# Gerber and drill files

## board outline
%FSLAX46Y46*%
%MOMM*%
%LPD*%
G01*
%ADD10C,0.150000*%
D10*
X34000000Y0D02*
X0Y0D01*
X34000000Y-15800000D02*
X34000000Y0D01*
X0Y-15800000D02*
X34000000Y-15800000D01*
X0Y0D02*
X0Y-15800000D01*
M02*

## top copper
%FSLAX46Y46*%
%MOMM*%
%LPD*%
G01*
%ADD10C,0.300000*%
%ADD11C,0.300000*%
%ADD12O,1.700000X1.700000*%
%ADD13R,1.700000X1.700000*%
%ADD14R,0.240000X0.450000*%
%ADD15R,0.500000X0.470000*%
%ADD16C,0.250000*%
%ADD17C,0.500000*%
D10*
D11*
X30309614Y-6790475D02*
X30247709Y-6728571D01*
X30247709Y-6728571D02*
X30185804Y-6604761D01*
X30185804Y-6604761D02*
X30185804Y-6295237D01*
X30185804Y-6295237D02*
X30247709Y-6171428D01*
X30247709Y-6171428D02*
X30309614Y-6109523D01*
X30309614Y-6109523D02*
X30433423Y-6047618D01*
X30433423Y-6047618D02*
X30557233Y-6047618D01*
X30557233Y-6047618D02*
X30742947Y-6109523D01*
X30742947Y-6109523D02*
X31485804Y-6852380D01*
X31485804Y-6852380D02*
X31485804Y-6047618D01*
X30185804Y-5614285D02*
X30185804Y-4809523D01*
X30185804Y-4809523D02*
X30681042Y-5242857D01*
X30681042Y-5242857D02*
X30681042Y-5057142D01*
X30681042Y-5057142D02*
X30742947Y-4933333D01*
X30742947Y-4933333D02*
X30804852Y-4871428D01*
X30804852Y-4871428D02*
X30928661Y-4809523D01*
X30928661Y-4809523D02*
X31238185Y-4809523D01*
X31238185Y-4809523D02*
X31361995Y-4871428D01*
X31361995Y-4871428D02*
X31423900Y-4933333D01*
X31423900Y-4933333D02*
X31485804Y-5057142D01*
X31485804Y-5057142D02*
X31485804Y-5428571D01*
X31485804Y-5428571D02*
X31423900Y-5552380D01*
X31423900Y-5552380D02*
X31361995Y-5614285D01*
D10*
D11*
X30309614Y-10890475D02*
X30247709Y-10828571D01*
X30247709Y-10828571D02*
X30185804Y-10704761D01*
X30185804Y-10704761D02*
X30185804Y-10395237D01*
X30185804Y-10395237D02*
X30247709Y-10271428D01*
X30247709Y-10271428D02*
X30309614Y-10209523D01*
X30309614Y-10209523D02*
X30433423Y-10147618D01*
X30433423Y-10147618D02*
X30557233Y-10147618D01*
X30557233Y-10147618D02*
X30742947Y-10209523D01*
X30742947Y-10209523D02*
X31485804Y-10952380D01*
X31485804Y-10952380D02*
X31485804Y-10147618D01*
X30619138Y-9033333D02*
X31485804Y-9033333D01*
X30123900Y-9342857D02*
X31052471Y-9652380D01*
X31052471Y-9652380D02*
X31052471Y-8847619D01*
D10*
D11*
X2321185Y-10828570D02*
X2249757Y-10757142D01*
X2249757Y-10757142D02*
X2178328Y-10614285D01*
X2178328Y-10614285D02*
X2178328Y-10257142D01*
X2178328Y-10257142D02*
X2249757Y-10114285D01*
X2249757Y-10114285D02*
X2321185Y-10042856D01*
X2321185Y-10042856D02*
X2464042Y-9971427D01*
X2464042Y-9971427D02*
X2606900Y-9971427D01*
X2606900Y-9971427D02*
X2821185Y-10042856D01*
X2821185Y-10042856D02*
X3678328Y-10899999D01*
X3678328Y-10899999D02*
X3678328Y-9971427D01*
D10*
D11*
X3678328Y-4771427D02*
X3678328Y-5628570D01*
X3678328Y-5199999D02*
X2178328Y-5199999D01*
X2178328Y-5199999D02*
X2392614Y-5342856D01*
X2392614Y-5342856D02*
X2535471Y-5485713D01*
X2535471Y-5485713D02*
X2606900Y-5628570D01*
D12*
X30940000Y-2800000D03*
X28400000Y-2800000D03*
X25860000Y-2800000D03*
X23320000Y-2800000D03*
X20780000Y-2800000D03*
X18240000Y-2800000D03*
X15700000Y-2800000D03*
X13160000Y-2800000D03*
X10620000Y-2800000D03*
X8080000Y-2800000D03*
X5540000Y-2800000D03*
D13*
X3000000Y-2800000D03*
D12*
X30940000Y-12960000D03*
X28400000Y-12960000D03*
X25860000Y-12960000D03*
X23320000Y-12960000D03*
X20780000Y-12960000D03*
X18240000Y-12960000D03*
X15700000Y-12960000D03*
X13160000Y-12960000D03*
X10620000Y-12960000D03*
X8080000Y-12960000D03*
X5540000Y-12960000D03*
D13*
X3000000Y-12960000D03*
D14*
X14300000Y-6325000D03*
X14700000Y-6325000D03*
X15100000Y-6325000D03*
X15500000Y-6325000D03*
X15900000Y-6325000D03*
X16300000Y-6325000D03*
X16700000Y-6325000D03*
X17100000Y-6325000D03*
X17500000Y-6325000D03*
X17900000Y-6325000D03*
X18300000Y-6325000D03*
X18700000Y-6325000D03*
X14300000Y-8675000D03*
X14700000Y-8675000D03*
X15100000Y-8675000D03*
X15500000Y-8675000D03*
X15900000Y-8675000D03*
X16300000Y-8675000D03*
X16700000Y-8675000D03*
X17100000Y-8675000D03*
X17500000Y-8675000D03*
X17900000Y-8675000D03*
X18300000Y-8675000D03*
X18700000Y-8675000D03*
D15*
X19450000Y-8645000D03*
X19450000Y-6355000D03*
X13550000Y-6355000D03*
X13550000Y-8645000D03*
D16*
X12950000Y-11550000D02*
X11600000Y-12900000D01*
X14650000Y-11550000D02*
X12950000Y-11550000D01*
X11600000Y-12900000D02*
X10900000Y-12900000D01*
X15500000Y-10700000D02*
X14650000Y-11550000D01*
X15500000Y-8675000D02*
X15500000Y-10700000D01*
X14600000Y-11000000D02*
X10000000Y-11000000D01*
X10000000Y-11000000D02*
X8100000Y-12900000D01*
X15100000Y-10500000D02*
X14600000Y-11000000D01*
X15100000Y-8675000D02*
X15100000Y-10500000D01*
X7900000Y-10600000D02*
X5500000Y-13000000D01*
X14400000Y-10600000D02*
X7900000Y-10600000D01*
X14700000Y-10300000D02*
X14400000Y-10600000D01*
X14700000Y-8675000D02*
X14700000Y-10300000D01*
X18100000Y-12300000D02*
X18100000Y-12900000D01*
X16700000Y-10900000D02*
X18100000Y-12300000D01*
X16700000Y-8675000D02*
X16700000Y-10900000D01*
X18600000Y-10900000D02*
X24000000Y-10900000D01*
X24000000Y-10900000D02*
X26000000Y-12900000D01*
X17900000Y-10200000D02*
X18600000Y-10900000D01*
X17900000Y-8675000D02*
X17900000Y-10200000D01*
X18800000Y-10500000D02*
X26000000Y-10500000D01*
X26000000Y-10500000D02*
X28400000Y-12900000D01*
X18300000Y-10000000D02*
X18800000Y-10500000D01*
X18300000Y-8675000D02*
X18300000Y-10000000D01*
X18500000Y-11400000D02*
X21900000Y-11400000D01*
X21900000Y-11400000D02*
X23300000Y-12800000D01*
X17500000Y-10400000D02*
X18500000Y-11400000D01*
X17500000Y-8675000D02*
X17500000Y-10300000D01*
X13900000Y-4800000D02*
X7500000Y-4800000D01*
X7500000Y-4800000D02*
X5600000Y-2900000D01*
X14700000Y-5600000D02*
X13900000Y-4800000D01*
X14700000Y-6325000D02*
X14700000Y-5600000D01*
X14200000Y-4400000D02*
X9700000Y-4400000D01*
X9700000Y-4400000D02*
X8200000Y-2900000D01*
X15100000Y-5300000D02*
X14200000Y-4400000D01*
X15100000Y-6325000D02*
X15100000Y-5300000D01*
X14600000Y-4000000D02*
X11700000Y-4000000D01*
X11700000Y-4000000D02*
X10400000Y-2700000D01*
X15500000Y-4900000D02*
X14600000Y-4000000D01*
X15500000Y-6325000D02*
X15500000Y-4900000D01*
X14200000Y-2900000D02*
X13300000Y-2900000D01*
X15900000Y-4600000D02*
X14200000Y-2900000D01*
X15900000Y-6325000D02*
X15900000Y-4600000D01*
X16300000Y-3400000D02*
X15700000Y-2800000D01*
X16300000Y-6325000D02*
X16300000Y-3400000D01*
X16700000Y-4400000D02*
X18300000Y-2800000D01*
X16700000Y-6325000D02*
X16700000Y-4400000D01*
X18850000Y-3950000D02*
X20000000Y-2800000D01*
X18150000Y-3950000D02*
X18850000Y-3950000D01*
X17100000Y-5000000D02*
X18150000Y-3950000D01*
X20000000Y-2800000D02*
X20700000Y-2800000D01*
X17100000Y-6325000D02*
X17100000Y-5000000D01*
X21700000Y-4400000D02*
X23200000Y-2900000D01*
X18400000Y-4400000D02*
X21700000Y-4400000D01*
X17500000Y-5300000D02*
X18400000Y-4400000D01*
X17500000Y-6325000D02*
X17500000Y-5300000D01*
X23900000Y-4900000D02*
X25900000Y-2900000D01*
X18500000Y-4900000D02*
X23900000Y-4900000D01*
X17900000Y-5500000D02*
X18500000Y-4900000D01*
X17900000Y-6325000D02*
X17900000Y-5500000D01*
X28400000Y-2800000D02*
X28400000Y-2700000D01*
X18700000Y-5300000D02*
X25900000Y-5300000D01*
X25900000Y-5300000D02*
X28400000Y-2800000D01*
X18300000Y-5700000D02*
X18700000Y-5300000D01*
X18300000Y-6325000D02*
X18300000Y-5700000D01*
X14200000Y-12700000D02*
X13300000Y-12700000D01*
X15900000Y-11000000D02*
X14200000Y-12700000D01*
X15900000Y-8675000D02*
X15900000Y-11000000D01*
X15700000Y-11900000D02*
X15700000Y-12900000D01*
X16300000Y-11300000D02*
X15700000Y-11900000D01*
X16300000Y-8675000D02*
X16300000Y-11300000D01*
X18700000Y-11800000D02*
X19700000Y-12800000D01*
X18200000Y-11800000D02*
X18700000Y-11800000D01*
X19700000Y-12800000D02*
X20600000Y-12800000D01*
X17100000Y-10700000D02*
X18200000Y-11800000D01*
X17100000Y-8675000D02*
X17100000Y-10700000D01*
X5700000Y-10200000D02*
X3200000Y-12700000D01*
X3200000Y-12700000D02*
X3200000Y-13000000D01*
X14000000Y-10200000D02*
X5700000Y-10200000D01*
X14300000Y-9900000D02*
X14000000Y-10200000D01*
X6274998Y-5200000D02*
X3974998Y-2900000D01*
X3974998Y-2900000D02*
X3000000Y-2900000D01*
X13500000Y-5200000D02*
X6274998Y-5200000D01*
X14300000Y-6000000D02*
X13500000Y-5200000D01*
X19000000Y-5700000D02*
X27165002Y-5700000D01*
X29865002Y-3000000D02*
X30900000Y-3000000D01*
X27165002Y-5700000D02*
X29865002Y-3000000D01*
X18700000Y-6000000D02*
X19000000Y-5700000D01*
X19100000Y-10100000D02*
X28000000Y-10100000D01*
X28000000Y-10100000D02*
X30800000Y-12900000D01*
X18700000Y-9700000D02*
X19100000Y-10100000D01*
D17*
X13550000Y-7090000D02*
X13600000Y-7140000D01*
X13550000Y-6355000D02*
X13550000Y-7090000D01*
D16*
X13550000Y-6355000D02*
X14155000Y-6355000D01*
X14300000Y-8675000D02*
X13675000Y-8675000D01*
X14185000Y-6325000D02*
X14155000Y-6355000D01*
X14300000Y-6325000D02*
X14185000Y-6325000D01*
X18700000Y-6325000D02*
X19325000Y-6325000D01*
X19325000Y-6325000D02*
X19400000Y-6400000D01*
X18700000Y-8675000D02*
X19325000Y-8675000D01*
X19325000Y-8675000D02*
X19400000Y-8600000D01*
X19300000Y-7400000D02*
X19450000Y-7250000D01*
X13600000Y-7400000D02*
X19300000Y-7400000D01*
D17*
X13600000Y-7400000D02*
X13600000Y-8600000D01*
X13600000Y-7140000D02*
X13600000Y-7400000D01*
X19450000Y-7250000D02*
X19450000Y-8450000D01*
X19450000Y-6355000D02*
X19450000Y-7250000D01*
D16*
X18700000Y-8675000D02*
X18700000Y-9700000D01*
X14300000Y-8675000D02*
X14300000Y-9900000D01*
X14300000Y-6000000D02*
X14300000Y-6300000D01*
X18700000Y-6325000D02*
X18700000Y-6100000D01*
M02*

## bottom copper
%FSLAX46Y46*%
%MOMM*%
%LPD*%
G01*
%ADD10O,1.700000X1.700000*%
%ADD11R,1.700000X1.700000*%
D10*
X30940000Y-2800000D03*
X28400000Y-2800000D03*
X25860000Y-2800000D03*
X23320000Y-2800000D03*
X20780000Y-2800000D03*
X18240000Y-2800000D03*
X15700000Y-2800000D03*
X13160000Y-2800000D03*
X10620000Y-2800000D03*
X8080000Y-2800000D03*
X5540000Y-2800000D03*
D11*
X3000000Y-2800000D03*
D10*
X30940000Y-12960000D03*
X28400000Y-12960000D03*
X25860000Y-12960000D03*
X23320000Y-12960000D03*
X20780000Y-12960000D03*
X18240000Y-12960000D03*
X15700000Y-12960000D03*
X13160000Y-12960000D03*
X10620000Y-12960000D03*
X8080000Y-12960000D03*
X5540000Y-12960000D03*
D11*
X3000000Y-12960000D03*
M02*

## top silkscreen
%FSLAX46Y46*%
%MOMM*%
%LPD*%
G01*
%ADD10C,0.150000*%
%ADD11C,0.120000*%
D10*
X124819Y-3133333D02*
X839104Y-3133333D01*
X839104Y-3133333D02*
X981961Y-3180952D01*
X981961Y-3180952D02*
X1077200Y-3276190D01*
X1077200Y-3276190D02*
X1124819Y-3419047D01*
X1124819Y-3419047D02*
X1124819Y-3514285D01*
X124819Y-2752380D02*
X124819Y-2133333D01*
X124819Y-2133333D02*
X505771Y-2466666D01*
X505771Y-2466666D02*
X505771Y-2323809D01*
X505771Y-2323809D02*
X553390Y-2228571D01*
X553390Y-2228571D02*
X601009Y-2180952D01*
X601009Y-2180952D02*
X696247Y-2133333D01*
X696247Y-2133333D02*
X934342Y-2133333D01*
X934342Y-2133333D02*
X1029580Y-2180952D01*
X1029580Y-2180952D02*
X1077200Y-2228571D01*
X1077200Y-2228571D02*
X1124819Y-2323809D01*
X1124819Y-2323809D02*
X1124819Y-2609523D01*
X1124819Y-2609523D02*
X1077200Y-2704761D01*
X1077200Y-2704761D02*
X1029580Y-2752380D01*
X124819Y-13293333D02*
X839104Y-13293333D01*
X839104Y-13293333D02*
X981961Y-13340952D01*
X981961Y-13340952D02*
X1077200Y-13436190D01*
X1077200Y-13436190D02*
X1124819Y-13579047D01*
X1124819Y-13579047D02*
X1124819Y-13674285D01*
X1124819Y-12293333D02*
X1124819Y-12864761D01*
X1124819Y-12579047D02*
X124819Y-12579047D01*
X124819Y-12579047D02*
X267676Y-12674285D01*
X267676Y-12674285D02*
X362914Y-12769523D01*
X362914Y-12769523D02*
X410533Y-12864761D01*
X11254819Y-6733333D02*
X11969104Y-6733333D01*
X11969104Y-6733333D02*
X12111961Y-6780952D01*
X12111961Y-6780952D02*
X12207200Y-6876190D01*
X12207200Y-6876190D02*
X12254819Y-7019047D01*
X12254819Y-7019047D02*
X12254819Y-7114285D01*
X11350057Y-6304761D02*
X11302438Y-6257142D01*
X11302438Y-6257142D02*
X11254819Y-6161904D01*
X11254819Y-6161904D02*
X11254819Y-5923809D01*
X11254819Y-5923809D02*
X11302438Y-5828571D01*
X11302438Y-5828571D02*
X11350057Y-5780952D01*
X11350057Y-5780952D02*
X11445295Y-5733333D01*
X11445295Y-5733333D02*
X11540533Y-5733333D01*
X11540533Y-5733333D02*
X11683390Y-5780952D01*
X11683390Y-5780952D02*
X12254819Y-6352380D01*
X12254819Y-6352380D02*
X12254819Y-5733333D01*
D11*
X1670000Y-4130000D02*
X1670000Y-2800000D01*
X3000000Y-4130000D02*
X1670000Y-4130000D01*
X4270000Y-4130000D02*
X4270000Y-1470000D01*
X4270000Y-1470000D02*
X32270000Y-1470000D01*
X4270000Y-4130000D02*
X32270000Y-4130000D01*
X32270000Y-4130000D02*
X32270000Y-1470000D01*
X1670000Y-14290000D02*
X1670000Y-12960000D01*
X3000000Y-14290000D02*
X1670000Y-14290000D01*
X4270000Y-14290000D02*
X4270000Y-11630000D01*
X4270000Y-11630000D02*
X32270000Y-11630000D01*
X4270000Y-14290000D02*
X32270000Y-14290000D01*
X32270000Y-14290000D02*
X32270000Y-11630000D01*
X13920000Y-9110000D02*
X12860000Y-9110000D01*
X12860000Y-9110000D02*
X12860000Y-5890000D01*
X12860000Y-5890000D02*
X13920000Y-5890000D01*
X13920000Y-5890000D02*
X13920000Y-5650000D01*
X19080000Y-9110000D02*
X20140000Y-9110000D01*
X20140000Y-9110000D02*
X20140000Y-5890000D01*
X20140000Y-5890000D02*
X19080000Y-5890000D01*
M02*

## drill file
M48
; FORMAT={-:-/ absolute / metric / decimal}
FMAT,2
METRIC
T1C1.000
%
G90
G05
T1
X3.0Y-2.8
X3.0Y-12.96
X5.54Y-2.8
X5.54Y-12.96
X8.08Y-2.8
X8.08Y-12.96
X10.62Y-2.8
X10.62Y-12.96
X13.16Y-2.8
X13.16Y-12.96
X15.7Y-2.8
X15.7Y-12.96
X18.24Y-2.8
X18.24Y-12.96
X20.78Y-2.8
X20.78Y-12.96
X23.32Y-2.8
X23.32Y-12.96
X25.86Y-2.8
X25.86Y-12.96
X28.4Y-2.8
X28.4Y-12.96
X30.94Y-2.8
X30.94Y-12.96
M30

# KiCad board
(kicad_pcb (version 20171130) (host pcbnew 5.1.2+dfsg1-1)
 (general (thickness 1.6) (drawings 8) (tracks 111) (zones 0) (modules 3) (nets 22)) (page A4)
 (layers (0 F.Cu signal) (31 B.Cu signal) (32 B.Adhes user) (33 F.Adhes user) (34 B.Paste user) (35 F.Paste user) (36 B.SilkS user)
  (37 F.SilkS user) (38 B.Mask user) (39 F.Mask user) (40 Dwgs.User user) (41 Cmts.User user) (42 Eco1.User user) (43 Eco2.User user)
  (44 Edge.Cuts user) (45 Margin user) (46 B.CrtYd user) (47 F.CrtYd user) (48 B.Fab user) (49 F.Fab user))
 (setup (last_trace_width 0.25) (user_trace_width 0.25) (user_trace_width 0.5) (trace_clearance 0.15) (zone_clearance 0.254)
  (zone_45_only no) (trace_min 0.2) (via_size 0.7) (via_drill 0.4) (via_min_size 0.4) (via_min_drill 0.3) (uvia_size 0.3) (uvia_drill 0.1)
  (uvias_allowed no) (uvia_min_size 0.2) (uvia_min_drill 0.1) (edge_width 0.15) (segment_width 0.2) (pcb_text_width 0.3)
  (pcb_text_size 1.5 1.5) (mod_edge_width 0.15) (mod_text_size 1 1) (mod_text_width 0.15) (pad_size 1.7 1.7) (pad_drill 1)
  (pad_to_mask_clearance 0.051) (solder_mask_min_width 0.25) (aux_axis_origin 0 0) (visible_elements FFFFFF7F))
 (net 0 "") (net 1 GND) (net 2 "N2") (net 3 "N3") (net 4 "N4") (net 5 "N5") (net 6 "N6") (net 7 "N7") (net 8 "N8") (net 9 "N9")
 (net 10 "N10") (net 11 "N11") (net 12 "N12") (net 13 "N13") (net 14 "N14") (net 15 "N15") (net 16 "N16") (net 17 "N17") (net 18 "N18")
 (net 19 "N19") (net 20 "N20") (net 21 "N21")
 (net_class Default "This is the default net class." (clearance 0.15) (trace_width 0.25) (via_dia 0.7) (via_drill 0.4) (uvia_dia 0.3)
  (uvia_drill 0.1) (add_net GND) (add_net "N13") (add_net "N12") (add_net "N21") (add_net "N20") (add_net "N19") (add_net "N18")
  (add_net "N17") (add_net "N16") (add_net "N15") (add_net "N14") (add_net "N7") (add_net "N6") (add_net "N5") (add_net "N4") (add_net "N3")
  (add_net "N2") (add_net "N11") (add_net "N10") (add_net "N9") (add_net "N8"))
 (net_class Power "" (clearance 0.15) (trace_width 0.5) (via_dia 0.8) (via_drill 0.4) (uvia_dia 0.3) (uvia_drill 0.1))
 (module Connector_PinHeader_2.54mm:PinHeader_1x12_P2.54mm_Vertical (layer F.Cu) (at 3 2.8 90)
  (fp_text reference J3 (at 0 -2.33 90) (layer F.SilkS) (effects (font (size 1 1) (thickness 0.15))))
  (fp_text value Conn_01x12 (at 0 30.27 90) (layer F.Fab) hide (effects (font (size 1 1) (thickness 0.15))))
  (fp_line (start -1.33 -1.33) (end 0 -1.33) (layer F.SilkS) (width 0.12))
  (fp_line (start -1.33 0) (end -1.33 -1.33) (layer F.SilkS) (width 0.12))
  (fp_line (start -1.33 1.27) (end 1.33 1.27) (layer F.SilkS) (width 0.12))
  (fp_line (start 1.33 1.27) (end 1.33 29.27) (layer F.SilkS) (width 0.12))
  (fp_line (start -1.33 1.27) (end -1.33 29.27) (layer F.SilkS) (width 0.12))
  (fp_line (start -1.33 29.27) (end 1.33 29.27) (layer F.SilkS) (width 0.12))
  (pad 12 thru_hole oval (at 0 27.94 90) (size 1.7 1.7) (drill 1) (layers *.Cu *.Mask) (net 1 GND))
  (pad 11 thru_hole oval (at 0 25.4 90) (size 1.7 1.7) (drill 1) (layers *.Cu *.Mask) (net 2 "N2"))
  (pad 10 thru_hole oval (at 0 22.86 90) (size 1.7 1.7) (drill 1) (layers *.Cu *.Mask) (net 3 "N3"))
  (pad 9 thru_hole oval (at 0 20.32 90) (size 1.7 1.7) (drill 1) (layers *.Cu *.Mask) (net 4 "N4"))
  (pad 8 thru_hole oval (at 0 17.78 90) (size 1.7 1.7) (drill 1) (layers *.Cu *.Mask) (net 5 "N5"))
  (pad 7 thru_hole oval (at 0 15.24 90) (size 1.7 1.7) (drill 1) (layers *.Cu *.Mask) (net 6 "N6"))
  (pad 6 thru_hole oval (at 0 12.7 90) (size 1.7 1.7) (drill 1) (layers *.Cu *.Mask) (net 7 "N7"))
  (pad 5 thru_hole oval (at 0 10.16 90) (size 1.7 1.7) (drill 1) (layers *.Cu *.Mask) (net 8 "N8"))
  (pad 4 thru_hole oval (at 0 7.62 90) (size 1.7 1.7) (drill 1) (layers *.Cu *.Mask) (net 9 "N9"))
  (pad 3 thru_hole oval (at 0 5.08 90) (size 1.7 1.7) (drill 1) (layers *.Cu *.Mask) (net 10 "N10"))
  (pad 2 thru_hole oval (at 0 2.54 90) (size 1.7 1.7) (drill 1) (layers *.Cu *.Mask) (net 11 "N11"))
  (pad 1 thru_hole rect (at 0 0 90) (size 1.7 1.7) (drill 1) (layers *.Cu *.Mask) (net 1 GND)))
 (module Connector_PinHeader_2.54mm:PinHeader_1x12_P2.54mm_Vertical (layer F.Cu) (at 3 12.96 90)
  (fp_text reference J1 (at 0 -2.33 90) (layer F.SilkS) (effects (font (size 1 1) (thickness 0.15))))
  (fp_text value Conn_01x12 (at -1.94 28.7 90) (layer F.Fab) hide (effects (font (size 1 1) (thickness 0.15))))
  (fp_line (start -1.33 -1.33) (end 0 -1.33) (layer F.SilkS) (width 0.12))
  (fp_line (start -1.33 0) (end -1.33 -1.33) (layer F.SilkS) (width 0.12))
  (fp_line (start -1.33 1.27) (end 1.33 1.27) (layer F.SilkS) (width 0.12))
  (fp_line (start 1.33 1.27) (end 1.33 29.27) (layer F.SilkS) (width 0.12))
  (fp_line (start -1.33 1.27) (end -1.33 29.27) (layer F.SilkS) (width 0.12))
  (fp_line (start -1.33 29.27) (end 1.33 29.27) (layer F.SilkS) (width 0.12))
  (pad 12 thru_hole oval (at 0 27.94 90) (size 1.7 1.7) (drill 1) (layers *.Cu *.Mask) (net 1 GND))
  (pad 11 thru_hole oval (at 0 25.4 90) (size 1.7 1.7) (drill 1) (layers *.Cu *.Mask) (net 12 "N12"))
  (pad 10 thru_hole oval (at 0 22.86 90) (size 1.7 1.7) (drill 1) (layers *.Cu *.Mask) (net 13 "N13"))
  (pad 9 thru_hole oval (at 0 20.32 90) (size 1.7 1.7) (drill 1) (layers *.Cu *.Mask) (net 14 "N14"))
  (pad 8 thru_hole oval (at 0 17.78 90) (size 1.7 1.7) (drill 1) (layers *.Cu *.Mask) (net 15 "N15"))
  (pad 7 thru_hole oval (at 0 15.24 90) (size 1.7 1.7) (drill 1) (layers *.Cu *.Mask) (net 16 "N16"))
  (pad 6 thru_hole oval (at 0 12.7 90) (size 1.7 1.7) (drill 1) (layers *.Cu *.Mask) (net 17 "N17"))
  (pad 5 thru_hole oval (at 0 10.16 90) (size 1.7 1.7) (drill 1) (layers *.Cu *.Mask) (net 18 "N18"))
  (pad 4 thru_hole oval (at 0 7.62 90) (size 1.7 1.7) (drill 1) (layers *.Cu *.Mask) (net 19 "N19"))
  (pad 3 thru_hole oval (at 0 5.08 90) (size 1.7 1.7) (drill 1) (layers *.Cu *.Mask) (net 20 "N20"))
  (pad 2 thru_hole oval (at 0 2.54 90) (size 1.7 1.7) (drill 1) (layers *.Cu *.Mask) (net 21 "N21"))
  (pad 1 thru_hole rect (at 0 0 90) (size 1.7 1.7) (drill 1) (layers *.Cu *.Mask) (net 1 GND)))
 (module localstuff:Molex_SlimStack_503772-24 (layer F.Cu) (at 16.5 7.5)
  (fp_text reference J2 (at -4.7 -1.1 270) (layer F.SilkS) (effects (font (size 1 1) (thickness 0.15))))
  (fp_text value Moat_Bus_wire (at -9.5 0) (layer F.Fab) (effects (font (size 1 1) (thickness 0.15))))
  (fp_line (start -2.58 1.61) (end -3.64 1.61) (layer F.SilkS) (width 0.12))
  (fp_line (start -3.64 1.61) (end -3.64 -1.61) (layer F.SilkS) (width 0.12))
  (fp_line (start -3.64 -1.61) (end -2.58 -1.61) (layer F.SilkS) (width 0.12))
  (fp_line (start -2.58 -1.61) (end -2.58 -1.85) (layer F.SilkS) (width 0.12))
  (fp_line (start 2.58 1.61) (end 3.64 1.61) (layer F.SilkS) (width 0.12))
  (fp_line (start 3.64 1.61) (end 3.64 -1.61) (layer F.SilkS) (width 0.12))
  (fp_line (start 3.64 -1.61) (end 2.58 -1.61) (layer F.SilkS) (width 0.12))
  (pad 1 smd rect (at -2.2 -1.175) (size 0.24 0.45) (layers F.Cu F.Paste F.Mask) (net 1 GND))
  (pad 3 smd rect (at -1.8 -1.175) (size 0.24 0.45) (layers F.Cu F.Paste F.Mask) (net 11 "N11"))
  (pad 5 smd rect (at -1.4 -1.175) (size 0.24 0.45) (layers F.Cu F.Paste F.Mask) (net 10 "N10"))
  (pad 7 smd rect (at -1 -1.175) (size 0.24 0.45) (layers F.Cu F.Paste F.Mask) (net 9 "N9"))
  (pad 9 smd rect (at -0.6 -1.175) (size 0.24 0.45) (layers F.Cu F.Paste F.Mask) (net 8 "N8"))
  (pad 11 smd rect (at -0.2 -1.175) (size 0.24 0.45) (layers F.Cu F.Paste F.Mask) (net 7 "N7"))
  (pad 13 smd rect (at 0.2 -1.175) (size 0.24 0.45) (layers F.Cu F.Paste F.Mask) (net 6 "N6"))
  (pad 15 smd rect (at 0.6 -1.175) (size 0.24 0.45) (layers F.Cu F.Paste F.Mask) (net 5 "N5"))
  (pad 17 smd rect (at 1 -1.175) (size 0.24 0.45) (layers F.Cu F.Paste F.Mask) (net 4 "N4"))
  (pad 19 smd rect (at 1.4 -1.175) (size 0.24 0.45) (layers F.Cu F.Paste F.Mask) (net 3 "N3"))
  (pad 21 smd rect (at 1.8 -1.175) (size 0.24 0.45) (layers F.Cu F.Paste F.Mask) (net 2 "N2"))
  (pad 23 smd rect (at 2.2 -1.175) (size 0.24 0.45) (layers F.Cu F.Paste F.Mask) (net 1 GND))
  (pad 2 smd rect (at -2.2 1.175) (size 0.24 0.45) (layers F.Cu F.Paste F.Mask) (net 1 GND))
  (pad 4 smd rect (at -1.8 1.175) (size 0.24 0.45) (layers F.Cu F.Paste F.Mask) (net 21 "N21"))
  (pad 6 smd rect (at -1.4 1.175) (size 0.24 0.45) (layers F.Cu F.Paste F.Mask) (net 20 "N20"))
  (pad 8 smd rect (at -1 1.175) (size 0.24 0.45) (layers F.Cu F.Paste F.Mask) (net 19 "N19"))
  (pad 10 smd rect (at -0.6 1.175) (size 0.24 0.45) (layers F.Cu F.Paste F.Mask) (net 18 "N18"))
  (pad 12 smd rect (at -0.2 1.175) (size 0.24 0.45) (layers F.Cu F.Paste F.Mask) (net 17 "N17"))
  (pad 14 smd rect (at 0.2 1.175) (size 0.24 0.45) (layers F.Cu F.Paste F.Mask) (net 16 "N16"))
  (pad 16 smd rect (at 0.6 1.175) (size 0.24 0.45) (layers F.Cu F.Paste F.Mask) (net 15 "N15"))
  (pad 18 smd rect (at 1 1.175) (size 0.24 0.45) (layers F.Cu F.Paste F.Mask) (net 14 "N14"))
  (pad 20 smd rect (at 1.4 1.175) (size 0.24 0.45) (layers F.Cu F.Paste F.Mask) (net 13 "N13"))
  (pad 22 smd rect (at 1.8 1.175) (size 0.24 0.45) (layers F.Cu F.Paste F.Mask) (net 12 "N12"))
  (pad 24 smd rect (at 2.2 1.175) (size 0.24 0.45) (layers F.Cu F.Paste F.Mask) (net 1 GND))
  (pad MP smd rect (at 2.95 1.145) (size 0.5 0.47) (layers F.Cu F.Paste F.Mask) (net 1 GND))
  (pad MP smd rect (at 2.95 -1.145) (size 0.5 0.47) (layers F.Cu F.Paste F.Mask) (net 1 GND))
  (pad MP smd rect (at -2.95 -1.145) (size 0.5 0.47) (layers F.Cu F.Paste F.Mask) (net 1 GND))
  (pad MP smd rect (at -2.95 1.145) (size 0.5 0.47) (layers F.Cu F.Paste F.Mask) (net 1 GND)))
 (gr_line (start 34 0) (end 0 0) (layer Edge.Cuts) (width 0.15))
 (gr_line (start 34 15.8) (end 34 0) (layer Edge.Cuts) (width 0.15))
 (gr_line (start 0 15.8) (end 34 15.8) (layer Edge.Cuts) (width 0.15))
 (gr_line (start 0 0) (end 0 15.8) (layer Edge.Cuts) (width 0.15))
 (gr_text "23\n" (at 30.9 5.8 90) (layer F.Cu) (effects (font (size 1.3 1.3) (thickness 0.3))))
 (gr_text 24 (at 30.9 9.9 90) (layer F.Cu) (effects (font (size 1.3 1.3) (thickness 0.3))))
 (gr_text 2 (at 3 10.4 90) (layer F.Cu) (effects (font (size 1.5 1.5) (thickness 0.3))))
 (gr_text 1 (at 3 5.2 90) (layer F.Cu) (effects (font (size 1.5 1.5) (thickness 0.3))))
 (segment (start 12.95 11.55) (end 11.6 12.9) (width 0.25) (layer F.Cu) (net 19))
 (segment (start 14.65 11.55) (end 12.95 11.55) (width 0.25) (layer F.Cu) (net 19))
 (segment (start 11.6 12.9) (end 10.9 12.9) (width 0.25) (layer F.Cu) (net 19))
 (segment (start 15.5 10.7) (end 14.65 11.55) (width 0.25) (layer F.Cu) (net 19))
 (segment (start 15.5 8.675) (end 15.5 10.7) (width 0.25) (layer F.Cu) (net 19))
 (segment (start 14.6 11) (end 10 11) (width 0.25) (layer F.Cu) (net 20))
 (segment (start 10 11) (end 8.1 12.9) (width 0.25) (layer F.Cu) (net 20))
 (segment (start 15.1 10.5) (end 14.6 11) (width 0.25) (layer F.Cu) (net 20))
 (segment (start 15.1 8.675) (end 15.1 10.5) (width 0.25) (layer F.Cu) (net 20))
 (segment (start 7.9 10.6) (end 5.5 13) (width 0.25) (layer F.Cu) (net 21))
 (segment (start 14.4 10.6) (end 7.9 10.6) (width 0.25) (layer F.Cu) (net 21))
 (segment (start 14.7 10.3) (end 14.4 10.6) (width 0.25) (layer F.Cu) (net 21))
 (segment (start 14.7 8.675) (end 14.7 10.3) (width 0.25) (layer F.Cu) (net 21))
 (segment (start 18.1 12.3) (end 18.1 12.9) (width 0.25) (layer F.Cu) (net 16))
 (segment (start 16.7 10.9) (end 18.1 12.3) (width 0.25) (layer F.Cu) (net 16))
 (segment (start 16.7 8.675) (end 16.7 10.9) (width 0.25) (layer F.Cu) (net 16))
 (segment (start 18.6 10.9) (end 24 10.9) (width 0.25) (layer F.Cu) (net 13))
 (segment (start 24 10.9) (end 26 12.9) (width 0.25) (layer F.Cu) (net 13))
 (segment (start 17.9 10.2) (end 18.6 10.9) (width 0.25) (layer F.Cu) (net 13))
 (segment (start 17.9 8.675) (end 17.9 10.2) (width 0.25) (layer F.Cu) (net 13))
 (segment (start 18.8 10.5) (end 26 10.5) (width 0.25) (layer F.Cu) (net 12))
 (segment (start 26 10.5) (end 28.4 12.9) (width 0.25) (layer F.Cu) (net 12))
 (segment (start 18.3 10) (end 18.8 10.5) (width 0.25) (layer F.Cu) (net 12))
 (segment (start 18.3 8.675) (end 18.3 10) (width 0.25) (layer F.Cu) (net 12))
 (segment (start 18.5 11.4) (end 21.9 11.4) (width 0.25) (layer F.Cu) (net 14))
 (segment (start 21.9 11.4) (end 23.3 12.8) (width 0.25) (layer F.Cu) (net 14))
 (segment (start 17.5 10.4) (end 18.5 11.4) (width 0.25) (layer F.Cu) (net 14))
 (segment (start 17.5 8.675) (end 17.5 10.3) (width 0.25) (layer F.Cu) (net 14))
 (segment (start 13.9 4.8) (end 7.5 4.8) (width 0.25) (layer F.Cu) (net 11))
 (segment (start 7.5 4.8) (end 5.6 2.9) (width 0.25) (layer F.Cu) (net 11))
 (segment (start 14.7 5.6) (end 13.9 4.8) (width 0.25) (layer F.Cu) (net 11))
 (segment (start 14.7 6.325) (end 14.7 5.6) (width 0.25) (layer F.Cu) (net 11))
 (segment (start 14.2 4.4) (end 9.7 4.4) (width 0.25) (layer F.Cu) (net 10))
 (segment (start 9.7 4.4) (end 8.2 2.9) (width 0.25) (layer F.Cu) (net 10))
 (segment (start 15.1 5.3) (end 14.2 4.4) (width 0.25) (layer F.Cu) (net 10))
 (segment (start 15.1 6.325) (end 15.1 5.3) (width 0.25) (layer F.Cu) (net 10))
 (segment (start 14.6 4) (end 11.7 4) (width 0.25) (layer F.Cu) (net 9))
 (segment (start 11.7 4) (end 10.4 2.7) (width 0.25) (layer F.Cu) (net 9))
 (segment (start 15.5 4.9) (end 14.6 4) (width 0.25) (layer F.Cu) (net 9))
 (segment (start 15.5 6.325) (end 15.5 4.9) (width 0.25) (layer F.Cu) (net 9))
 (segment (start 14.2 2.9) (end 13.3 2.9) (width 0.25) (layer F.Cu) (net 8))
 (segment (start 15.9 4.6) (end 14.2 2.9) (width 0.25) (layer F.Cu) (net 8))
 (segment (start 15.9 6.325) (end 15.9 4.6) (width 0.25) (layer F.Cu) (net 8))
 (segment (start 16.3 3.4) (end 15.7 2.8) (width 0.25) (layer F.Cu) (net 7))
 (segment (start 16.3 6.325) (end 16.3 3.4) (width 0.25) (layer F.Cu) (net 7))
 (segment (start 16.7 4.4) (end 18.3 2.8) (width 0.25) (layer F.Cu) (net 6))
 (segment (start 16.7 6.325) (end 16.7 4.4) (width 0.25) (layer F.Cu) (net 6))
 (segment (start 18.85 3.95) (end 20 2.8) (width 0.25) (layer F.Cu) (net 5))
 (segment (start 18.15 3.95) (end 18.85 3.95) (width 0.25) (layer F.Cu) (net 5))
 (segment (start 17.1 5) (end 18.15 3.95) (width 0.25) (layer F.Cu) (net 5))
 (segment (start 20 2.8) (end 20.7 2.8) (width 0.25) (layer F.Cu) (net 5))
 (segment (start 17.1 6.325) (end 17.1 5) (width 0.25) (layer F.Cu) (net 5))
 (segment (start 21.7 4.4) (end 23.2 2.9) (width 0.25) (layer F.Cu) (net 4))
 (segment (start 18.4 4.4) (end 21.7 4.4) (width 0.25) (layer F.Cu) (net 4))
 (segment (start 17.5 5.3) (end 18.4 4.4) (width 0.25) (layer F.Cu) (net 4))
 (segment (start 17.5 6.325) (end 17.5 5.3) (width 0.25) (layer F.Cu) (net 4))
 (segment (start 23.9 4.9) (end 25.9 2.9) (width 0.25) (layer F.Cu) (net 3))
 (segment (start 18.5 4.9) (end 23.9 4.9) (width 0.25) (layer F.Cu) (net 3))
 (segment (start 17.9 5.5) (end 18.5 4.9) (width 0.25) (layer F.Cu) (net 3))
 (segment (start 17.9 6.325) (end 17.9 5.5) (width 0.25) (layer F.Cu) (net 3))
 (segment (start 28.4 2.8) (end 28.4 2.7) (width 0.25) (layer F.Cu) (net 2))
 (segment (start 18.7 5.3) (end 25.9 5.3) (width 0.25) (layer F.Cu) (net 2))
 (segment (start 25.9 5.3) (end 28.4 2.8) (width 0.25) (layer F.Cu) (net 2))
 (segment (start 18.3 5.7) (end 18.7 5.3) (width 0.25) (layer F.Cu) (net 2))
 (segment (start 18.3 6.325) (end 18.3 5.7) (width 0.25) (layer F.Cu) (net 2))
 (segment (start 14.2 12.7) (end 13.3 12.7) (width 0.25) (layer F.Cu) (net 18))
 (segment (start 15.9 11) (end 14.2 12.7) (width 0.25) (layer F.Cu) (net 18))
 (segment (start 15.9 8.675) (end 15.9 11) (width 0.25) (layer F.Cu) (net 18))
 (segment (start 15.7 11.9) (end 15.7 12.9) (width 0.25) (layer F.Cu) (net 17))
 (segment (start 16.3 11.3) (end 15.7 11.9) (width 0.25) (layer F.Cu) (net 17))
 (segment (start 16.3 8.675) (end 16.3 11.3) (width 0.25) (layer F.Cu) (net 17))
 (segment (start 18.7 11.8) (end 19.7 12.8) (width 0.25) (layer F.Cu) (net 15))
 (segment (start 18.2 11.8) (end 18.7 11.8) (width 0.25) (layer F.Cu) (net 15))
 (segment (start 19.7 12.8) (end 20.6 12.8) (width 0.25) (layer F.Cu) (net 15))
 (segment (start 17.1 10.7) (end 18.2 11.8) (width 0.25) (layer F.Cu) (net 15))
 (segment (start 17.1 8.675) (end 17.1 10.7) (width 0.25) (layer F.Cu) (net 15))
 (segment (start 5.7 10.2) (end 3.2 12.7) (width 0.25) (layer F.Cu) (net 1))
 (segment (start 3.2 12.7) (end 3.2 13) (width 0.25) (layer F.Cu) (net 1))
 (segment (start 14 10.2) (end 5.7 10.2) (width 0.25) (layer F.Cu) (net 1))
 (segment (start 14.3 9.9) (end 14 10.2) (width 0.25) (layer F.Cu) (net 1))
 (segment (start 6.274998 5.2) (end 3.974998 2.9) (width 0.25) (layer F.Cu) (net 1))
 (segment (start 3.974998 2.9) (end 3 2.9) (width 0.25) (layer F.Cu) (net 1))
 (segment (start 13.5 5.2) (end 6.274998 5.2) (width 0.25) (layer F.Cu) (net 1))
 (segment (start 14.3 6) (end 13.5 5.2) (width 0.25) (layer F.Cu) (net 1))
 (segment (start 19 5.7) (end 27.165002 5.7) (width 0.25) (layer F.Cu) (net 1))
 (segment (start 29.865002 3) (end 30.9 3) (width 0.25) (layer F.Cu) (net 1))
 (segment (start 27.165002 5.7) (end 29.865002 3) (width 0.25) (layer F.Cu) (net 1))
 (segment (start 18.7 6) (end 19 5.7) (width 0.25) (layer F.Cu) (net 1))
 (segment (start 19.1 10.1) (end 28 10.1) (width 0.25) (layer F.Cu) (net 1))
 (segment (start 28 10.1) (end 30.8 12.9) (width 0.25) (layer F.Cu) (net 1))
 (segment (start 18.7 9.7) (end 19.1 10.1) (width 0.25) (layer F.Cu) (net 1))
 (segment (start 13.55 7.09) (end 13.6 7.14) (width 0.5) (layer F.Cu) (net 1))
 (segment (start 13.55 6.355) (end 13.55 7.09) (width 0.5) (layer F.Cu) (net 1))
 (segment (start 13.55 6.355) (end 14.155 6.355) (width 0.25) (layer F.Cu) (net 1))
 (segment (start 14.3 8.675) (end 13.675 8.675) (width 0.25) (layer F.Cu) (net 1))
 (segment (start 14.185 6.325) (end 14.155 6.355) (width 0.25) (layer F.Cu) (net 1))
 (segment (start 14.3 6.325) (end 14.185 6.325) (width 0.25) (layer F.Cu) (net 1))
 (segment (start 18.7 6.325) (end 19.325 6.325) (width 0.25) (layer F.Cu) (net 1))
 (segment (start 19.325 6.325) (end 19.4 6.4) (width 0.25) (layer F.Cu) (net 1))
 (segment (start 18.7 8.675) (end 19.325 8.675) (width 0.25) (layer F.Cu) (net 1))
 (segment (start 19.325 8.675) (end 19.4 8.6) (width 0.25) (layer F.Cu) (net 1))
 (segment (start 19.3 7.4) (end 19.45 7.25) (width 0.25) (layer F.Cu) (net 1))
 (segment (start 13.6 7.4) (end 19.3 7.4) (width 0.25) (layer F.Cu) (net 1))
 (segment (start 13.6 7.4) (end 13.6 8.6) (width 0.5) (layer F.Cu) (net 1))
 (segment (start 13.6 7.14) (end 13.6 7.4) (width 0.5) (layer F.Cu) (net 1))
 (segment (start 19.45 7.25) (end 19.45 8.45) (width 0.5) (layer F.Cu) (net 1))
 (segment (start 19.45 6.355) (end 19.45 7.25) (width 0.5) (layer F.Cu) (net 1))
 (segment (start 18.7 8.675) (end 18.7 9.7) (width 0.25) (layer F.Cu) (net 1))
 (segment (start 14.3 8.675) (end 14.3 9.9) (width 0.25) (layer F.Cu) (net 1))
 (segment (start 14.3 6) (end 14.3 6.3) (width 0.25) (layer F.Cu) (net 1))
 (segment (start 18.7 6.325) (end 18.7 6.1) (width 0.25) (layer F.Cu) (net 1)))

